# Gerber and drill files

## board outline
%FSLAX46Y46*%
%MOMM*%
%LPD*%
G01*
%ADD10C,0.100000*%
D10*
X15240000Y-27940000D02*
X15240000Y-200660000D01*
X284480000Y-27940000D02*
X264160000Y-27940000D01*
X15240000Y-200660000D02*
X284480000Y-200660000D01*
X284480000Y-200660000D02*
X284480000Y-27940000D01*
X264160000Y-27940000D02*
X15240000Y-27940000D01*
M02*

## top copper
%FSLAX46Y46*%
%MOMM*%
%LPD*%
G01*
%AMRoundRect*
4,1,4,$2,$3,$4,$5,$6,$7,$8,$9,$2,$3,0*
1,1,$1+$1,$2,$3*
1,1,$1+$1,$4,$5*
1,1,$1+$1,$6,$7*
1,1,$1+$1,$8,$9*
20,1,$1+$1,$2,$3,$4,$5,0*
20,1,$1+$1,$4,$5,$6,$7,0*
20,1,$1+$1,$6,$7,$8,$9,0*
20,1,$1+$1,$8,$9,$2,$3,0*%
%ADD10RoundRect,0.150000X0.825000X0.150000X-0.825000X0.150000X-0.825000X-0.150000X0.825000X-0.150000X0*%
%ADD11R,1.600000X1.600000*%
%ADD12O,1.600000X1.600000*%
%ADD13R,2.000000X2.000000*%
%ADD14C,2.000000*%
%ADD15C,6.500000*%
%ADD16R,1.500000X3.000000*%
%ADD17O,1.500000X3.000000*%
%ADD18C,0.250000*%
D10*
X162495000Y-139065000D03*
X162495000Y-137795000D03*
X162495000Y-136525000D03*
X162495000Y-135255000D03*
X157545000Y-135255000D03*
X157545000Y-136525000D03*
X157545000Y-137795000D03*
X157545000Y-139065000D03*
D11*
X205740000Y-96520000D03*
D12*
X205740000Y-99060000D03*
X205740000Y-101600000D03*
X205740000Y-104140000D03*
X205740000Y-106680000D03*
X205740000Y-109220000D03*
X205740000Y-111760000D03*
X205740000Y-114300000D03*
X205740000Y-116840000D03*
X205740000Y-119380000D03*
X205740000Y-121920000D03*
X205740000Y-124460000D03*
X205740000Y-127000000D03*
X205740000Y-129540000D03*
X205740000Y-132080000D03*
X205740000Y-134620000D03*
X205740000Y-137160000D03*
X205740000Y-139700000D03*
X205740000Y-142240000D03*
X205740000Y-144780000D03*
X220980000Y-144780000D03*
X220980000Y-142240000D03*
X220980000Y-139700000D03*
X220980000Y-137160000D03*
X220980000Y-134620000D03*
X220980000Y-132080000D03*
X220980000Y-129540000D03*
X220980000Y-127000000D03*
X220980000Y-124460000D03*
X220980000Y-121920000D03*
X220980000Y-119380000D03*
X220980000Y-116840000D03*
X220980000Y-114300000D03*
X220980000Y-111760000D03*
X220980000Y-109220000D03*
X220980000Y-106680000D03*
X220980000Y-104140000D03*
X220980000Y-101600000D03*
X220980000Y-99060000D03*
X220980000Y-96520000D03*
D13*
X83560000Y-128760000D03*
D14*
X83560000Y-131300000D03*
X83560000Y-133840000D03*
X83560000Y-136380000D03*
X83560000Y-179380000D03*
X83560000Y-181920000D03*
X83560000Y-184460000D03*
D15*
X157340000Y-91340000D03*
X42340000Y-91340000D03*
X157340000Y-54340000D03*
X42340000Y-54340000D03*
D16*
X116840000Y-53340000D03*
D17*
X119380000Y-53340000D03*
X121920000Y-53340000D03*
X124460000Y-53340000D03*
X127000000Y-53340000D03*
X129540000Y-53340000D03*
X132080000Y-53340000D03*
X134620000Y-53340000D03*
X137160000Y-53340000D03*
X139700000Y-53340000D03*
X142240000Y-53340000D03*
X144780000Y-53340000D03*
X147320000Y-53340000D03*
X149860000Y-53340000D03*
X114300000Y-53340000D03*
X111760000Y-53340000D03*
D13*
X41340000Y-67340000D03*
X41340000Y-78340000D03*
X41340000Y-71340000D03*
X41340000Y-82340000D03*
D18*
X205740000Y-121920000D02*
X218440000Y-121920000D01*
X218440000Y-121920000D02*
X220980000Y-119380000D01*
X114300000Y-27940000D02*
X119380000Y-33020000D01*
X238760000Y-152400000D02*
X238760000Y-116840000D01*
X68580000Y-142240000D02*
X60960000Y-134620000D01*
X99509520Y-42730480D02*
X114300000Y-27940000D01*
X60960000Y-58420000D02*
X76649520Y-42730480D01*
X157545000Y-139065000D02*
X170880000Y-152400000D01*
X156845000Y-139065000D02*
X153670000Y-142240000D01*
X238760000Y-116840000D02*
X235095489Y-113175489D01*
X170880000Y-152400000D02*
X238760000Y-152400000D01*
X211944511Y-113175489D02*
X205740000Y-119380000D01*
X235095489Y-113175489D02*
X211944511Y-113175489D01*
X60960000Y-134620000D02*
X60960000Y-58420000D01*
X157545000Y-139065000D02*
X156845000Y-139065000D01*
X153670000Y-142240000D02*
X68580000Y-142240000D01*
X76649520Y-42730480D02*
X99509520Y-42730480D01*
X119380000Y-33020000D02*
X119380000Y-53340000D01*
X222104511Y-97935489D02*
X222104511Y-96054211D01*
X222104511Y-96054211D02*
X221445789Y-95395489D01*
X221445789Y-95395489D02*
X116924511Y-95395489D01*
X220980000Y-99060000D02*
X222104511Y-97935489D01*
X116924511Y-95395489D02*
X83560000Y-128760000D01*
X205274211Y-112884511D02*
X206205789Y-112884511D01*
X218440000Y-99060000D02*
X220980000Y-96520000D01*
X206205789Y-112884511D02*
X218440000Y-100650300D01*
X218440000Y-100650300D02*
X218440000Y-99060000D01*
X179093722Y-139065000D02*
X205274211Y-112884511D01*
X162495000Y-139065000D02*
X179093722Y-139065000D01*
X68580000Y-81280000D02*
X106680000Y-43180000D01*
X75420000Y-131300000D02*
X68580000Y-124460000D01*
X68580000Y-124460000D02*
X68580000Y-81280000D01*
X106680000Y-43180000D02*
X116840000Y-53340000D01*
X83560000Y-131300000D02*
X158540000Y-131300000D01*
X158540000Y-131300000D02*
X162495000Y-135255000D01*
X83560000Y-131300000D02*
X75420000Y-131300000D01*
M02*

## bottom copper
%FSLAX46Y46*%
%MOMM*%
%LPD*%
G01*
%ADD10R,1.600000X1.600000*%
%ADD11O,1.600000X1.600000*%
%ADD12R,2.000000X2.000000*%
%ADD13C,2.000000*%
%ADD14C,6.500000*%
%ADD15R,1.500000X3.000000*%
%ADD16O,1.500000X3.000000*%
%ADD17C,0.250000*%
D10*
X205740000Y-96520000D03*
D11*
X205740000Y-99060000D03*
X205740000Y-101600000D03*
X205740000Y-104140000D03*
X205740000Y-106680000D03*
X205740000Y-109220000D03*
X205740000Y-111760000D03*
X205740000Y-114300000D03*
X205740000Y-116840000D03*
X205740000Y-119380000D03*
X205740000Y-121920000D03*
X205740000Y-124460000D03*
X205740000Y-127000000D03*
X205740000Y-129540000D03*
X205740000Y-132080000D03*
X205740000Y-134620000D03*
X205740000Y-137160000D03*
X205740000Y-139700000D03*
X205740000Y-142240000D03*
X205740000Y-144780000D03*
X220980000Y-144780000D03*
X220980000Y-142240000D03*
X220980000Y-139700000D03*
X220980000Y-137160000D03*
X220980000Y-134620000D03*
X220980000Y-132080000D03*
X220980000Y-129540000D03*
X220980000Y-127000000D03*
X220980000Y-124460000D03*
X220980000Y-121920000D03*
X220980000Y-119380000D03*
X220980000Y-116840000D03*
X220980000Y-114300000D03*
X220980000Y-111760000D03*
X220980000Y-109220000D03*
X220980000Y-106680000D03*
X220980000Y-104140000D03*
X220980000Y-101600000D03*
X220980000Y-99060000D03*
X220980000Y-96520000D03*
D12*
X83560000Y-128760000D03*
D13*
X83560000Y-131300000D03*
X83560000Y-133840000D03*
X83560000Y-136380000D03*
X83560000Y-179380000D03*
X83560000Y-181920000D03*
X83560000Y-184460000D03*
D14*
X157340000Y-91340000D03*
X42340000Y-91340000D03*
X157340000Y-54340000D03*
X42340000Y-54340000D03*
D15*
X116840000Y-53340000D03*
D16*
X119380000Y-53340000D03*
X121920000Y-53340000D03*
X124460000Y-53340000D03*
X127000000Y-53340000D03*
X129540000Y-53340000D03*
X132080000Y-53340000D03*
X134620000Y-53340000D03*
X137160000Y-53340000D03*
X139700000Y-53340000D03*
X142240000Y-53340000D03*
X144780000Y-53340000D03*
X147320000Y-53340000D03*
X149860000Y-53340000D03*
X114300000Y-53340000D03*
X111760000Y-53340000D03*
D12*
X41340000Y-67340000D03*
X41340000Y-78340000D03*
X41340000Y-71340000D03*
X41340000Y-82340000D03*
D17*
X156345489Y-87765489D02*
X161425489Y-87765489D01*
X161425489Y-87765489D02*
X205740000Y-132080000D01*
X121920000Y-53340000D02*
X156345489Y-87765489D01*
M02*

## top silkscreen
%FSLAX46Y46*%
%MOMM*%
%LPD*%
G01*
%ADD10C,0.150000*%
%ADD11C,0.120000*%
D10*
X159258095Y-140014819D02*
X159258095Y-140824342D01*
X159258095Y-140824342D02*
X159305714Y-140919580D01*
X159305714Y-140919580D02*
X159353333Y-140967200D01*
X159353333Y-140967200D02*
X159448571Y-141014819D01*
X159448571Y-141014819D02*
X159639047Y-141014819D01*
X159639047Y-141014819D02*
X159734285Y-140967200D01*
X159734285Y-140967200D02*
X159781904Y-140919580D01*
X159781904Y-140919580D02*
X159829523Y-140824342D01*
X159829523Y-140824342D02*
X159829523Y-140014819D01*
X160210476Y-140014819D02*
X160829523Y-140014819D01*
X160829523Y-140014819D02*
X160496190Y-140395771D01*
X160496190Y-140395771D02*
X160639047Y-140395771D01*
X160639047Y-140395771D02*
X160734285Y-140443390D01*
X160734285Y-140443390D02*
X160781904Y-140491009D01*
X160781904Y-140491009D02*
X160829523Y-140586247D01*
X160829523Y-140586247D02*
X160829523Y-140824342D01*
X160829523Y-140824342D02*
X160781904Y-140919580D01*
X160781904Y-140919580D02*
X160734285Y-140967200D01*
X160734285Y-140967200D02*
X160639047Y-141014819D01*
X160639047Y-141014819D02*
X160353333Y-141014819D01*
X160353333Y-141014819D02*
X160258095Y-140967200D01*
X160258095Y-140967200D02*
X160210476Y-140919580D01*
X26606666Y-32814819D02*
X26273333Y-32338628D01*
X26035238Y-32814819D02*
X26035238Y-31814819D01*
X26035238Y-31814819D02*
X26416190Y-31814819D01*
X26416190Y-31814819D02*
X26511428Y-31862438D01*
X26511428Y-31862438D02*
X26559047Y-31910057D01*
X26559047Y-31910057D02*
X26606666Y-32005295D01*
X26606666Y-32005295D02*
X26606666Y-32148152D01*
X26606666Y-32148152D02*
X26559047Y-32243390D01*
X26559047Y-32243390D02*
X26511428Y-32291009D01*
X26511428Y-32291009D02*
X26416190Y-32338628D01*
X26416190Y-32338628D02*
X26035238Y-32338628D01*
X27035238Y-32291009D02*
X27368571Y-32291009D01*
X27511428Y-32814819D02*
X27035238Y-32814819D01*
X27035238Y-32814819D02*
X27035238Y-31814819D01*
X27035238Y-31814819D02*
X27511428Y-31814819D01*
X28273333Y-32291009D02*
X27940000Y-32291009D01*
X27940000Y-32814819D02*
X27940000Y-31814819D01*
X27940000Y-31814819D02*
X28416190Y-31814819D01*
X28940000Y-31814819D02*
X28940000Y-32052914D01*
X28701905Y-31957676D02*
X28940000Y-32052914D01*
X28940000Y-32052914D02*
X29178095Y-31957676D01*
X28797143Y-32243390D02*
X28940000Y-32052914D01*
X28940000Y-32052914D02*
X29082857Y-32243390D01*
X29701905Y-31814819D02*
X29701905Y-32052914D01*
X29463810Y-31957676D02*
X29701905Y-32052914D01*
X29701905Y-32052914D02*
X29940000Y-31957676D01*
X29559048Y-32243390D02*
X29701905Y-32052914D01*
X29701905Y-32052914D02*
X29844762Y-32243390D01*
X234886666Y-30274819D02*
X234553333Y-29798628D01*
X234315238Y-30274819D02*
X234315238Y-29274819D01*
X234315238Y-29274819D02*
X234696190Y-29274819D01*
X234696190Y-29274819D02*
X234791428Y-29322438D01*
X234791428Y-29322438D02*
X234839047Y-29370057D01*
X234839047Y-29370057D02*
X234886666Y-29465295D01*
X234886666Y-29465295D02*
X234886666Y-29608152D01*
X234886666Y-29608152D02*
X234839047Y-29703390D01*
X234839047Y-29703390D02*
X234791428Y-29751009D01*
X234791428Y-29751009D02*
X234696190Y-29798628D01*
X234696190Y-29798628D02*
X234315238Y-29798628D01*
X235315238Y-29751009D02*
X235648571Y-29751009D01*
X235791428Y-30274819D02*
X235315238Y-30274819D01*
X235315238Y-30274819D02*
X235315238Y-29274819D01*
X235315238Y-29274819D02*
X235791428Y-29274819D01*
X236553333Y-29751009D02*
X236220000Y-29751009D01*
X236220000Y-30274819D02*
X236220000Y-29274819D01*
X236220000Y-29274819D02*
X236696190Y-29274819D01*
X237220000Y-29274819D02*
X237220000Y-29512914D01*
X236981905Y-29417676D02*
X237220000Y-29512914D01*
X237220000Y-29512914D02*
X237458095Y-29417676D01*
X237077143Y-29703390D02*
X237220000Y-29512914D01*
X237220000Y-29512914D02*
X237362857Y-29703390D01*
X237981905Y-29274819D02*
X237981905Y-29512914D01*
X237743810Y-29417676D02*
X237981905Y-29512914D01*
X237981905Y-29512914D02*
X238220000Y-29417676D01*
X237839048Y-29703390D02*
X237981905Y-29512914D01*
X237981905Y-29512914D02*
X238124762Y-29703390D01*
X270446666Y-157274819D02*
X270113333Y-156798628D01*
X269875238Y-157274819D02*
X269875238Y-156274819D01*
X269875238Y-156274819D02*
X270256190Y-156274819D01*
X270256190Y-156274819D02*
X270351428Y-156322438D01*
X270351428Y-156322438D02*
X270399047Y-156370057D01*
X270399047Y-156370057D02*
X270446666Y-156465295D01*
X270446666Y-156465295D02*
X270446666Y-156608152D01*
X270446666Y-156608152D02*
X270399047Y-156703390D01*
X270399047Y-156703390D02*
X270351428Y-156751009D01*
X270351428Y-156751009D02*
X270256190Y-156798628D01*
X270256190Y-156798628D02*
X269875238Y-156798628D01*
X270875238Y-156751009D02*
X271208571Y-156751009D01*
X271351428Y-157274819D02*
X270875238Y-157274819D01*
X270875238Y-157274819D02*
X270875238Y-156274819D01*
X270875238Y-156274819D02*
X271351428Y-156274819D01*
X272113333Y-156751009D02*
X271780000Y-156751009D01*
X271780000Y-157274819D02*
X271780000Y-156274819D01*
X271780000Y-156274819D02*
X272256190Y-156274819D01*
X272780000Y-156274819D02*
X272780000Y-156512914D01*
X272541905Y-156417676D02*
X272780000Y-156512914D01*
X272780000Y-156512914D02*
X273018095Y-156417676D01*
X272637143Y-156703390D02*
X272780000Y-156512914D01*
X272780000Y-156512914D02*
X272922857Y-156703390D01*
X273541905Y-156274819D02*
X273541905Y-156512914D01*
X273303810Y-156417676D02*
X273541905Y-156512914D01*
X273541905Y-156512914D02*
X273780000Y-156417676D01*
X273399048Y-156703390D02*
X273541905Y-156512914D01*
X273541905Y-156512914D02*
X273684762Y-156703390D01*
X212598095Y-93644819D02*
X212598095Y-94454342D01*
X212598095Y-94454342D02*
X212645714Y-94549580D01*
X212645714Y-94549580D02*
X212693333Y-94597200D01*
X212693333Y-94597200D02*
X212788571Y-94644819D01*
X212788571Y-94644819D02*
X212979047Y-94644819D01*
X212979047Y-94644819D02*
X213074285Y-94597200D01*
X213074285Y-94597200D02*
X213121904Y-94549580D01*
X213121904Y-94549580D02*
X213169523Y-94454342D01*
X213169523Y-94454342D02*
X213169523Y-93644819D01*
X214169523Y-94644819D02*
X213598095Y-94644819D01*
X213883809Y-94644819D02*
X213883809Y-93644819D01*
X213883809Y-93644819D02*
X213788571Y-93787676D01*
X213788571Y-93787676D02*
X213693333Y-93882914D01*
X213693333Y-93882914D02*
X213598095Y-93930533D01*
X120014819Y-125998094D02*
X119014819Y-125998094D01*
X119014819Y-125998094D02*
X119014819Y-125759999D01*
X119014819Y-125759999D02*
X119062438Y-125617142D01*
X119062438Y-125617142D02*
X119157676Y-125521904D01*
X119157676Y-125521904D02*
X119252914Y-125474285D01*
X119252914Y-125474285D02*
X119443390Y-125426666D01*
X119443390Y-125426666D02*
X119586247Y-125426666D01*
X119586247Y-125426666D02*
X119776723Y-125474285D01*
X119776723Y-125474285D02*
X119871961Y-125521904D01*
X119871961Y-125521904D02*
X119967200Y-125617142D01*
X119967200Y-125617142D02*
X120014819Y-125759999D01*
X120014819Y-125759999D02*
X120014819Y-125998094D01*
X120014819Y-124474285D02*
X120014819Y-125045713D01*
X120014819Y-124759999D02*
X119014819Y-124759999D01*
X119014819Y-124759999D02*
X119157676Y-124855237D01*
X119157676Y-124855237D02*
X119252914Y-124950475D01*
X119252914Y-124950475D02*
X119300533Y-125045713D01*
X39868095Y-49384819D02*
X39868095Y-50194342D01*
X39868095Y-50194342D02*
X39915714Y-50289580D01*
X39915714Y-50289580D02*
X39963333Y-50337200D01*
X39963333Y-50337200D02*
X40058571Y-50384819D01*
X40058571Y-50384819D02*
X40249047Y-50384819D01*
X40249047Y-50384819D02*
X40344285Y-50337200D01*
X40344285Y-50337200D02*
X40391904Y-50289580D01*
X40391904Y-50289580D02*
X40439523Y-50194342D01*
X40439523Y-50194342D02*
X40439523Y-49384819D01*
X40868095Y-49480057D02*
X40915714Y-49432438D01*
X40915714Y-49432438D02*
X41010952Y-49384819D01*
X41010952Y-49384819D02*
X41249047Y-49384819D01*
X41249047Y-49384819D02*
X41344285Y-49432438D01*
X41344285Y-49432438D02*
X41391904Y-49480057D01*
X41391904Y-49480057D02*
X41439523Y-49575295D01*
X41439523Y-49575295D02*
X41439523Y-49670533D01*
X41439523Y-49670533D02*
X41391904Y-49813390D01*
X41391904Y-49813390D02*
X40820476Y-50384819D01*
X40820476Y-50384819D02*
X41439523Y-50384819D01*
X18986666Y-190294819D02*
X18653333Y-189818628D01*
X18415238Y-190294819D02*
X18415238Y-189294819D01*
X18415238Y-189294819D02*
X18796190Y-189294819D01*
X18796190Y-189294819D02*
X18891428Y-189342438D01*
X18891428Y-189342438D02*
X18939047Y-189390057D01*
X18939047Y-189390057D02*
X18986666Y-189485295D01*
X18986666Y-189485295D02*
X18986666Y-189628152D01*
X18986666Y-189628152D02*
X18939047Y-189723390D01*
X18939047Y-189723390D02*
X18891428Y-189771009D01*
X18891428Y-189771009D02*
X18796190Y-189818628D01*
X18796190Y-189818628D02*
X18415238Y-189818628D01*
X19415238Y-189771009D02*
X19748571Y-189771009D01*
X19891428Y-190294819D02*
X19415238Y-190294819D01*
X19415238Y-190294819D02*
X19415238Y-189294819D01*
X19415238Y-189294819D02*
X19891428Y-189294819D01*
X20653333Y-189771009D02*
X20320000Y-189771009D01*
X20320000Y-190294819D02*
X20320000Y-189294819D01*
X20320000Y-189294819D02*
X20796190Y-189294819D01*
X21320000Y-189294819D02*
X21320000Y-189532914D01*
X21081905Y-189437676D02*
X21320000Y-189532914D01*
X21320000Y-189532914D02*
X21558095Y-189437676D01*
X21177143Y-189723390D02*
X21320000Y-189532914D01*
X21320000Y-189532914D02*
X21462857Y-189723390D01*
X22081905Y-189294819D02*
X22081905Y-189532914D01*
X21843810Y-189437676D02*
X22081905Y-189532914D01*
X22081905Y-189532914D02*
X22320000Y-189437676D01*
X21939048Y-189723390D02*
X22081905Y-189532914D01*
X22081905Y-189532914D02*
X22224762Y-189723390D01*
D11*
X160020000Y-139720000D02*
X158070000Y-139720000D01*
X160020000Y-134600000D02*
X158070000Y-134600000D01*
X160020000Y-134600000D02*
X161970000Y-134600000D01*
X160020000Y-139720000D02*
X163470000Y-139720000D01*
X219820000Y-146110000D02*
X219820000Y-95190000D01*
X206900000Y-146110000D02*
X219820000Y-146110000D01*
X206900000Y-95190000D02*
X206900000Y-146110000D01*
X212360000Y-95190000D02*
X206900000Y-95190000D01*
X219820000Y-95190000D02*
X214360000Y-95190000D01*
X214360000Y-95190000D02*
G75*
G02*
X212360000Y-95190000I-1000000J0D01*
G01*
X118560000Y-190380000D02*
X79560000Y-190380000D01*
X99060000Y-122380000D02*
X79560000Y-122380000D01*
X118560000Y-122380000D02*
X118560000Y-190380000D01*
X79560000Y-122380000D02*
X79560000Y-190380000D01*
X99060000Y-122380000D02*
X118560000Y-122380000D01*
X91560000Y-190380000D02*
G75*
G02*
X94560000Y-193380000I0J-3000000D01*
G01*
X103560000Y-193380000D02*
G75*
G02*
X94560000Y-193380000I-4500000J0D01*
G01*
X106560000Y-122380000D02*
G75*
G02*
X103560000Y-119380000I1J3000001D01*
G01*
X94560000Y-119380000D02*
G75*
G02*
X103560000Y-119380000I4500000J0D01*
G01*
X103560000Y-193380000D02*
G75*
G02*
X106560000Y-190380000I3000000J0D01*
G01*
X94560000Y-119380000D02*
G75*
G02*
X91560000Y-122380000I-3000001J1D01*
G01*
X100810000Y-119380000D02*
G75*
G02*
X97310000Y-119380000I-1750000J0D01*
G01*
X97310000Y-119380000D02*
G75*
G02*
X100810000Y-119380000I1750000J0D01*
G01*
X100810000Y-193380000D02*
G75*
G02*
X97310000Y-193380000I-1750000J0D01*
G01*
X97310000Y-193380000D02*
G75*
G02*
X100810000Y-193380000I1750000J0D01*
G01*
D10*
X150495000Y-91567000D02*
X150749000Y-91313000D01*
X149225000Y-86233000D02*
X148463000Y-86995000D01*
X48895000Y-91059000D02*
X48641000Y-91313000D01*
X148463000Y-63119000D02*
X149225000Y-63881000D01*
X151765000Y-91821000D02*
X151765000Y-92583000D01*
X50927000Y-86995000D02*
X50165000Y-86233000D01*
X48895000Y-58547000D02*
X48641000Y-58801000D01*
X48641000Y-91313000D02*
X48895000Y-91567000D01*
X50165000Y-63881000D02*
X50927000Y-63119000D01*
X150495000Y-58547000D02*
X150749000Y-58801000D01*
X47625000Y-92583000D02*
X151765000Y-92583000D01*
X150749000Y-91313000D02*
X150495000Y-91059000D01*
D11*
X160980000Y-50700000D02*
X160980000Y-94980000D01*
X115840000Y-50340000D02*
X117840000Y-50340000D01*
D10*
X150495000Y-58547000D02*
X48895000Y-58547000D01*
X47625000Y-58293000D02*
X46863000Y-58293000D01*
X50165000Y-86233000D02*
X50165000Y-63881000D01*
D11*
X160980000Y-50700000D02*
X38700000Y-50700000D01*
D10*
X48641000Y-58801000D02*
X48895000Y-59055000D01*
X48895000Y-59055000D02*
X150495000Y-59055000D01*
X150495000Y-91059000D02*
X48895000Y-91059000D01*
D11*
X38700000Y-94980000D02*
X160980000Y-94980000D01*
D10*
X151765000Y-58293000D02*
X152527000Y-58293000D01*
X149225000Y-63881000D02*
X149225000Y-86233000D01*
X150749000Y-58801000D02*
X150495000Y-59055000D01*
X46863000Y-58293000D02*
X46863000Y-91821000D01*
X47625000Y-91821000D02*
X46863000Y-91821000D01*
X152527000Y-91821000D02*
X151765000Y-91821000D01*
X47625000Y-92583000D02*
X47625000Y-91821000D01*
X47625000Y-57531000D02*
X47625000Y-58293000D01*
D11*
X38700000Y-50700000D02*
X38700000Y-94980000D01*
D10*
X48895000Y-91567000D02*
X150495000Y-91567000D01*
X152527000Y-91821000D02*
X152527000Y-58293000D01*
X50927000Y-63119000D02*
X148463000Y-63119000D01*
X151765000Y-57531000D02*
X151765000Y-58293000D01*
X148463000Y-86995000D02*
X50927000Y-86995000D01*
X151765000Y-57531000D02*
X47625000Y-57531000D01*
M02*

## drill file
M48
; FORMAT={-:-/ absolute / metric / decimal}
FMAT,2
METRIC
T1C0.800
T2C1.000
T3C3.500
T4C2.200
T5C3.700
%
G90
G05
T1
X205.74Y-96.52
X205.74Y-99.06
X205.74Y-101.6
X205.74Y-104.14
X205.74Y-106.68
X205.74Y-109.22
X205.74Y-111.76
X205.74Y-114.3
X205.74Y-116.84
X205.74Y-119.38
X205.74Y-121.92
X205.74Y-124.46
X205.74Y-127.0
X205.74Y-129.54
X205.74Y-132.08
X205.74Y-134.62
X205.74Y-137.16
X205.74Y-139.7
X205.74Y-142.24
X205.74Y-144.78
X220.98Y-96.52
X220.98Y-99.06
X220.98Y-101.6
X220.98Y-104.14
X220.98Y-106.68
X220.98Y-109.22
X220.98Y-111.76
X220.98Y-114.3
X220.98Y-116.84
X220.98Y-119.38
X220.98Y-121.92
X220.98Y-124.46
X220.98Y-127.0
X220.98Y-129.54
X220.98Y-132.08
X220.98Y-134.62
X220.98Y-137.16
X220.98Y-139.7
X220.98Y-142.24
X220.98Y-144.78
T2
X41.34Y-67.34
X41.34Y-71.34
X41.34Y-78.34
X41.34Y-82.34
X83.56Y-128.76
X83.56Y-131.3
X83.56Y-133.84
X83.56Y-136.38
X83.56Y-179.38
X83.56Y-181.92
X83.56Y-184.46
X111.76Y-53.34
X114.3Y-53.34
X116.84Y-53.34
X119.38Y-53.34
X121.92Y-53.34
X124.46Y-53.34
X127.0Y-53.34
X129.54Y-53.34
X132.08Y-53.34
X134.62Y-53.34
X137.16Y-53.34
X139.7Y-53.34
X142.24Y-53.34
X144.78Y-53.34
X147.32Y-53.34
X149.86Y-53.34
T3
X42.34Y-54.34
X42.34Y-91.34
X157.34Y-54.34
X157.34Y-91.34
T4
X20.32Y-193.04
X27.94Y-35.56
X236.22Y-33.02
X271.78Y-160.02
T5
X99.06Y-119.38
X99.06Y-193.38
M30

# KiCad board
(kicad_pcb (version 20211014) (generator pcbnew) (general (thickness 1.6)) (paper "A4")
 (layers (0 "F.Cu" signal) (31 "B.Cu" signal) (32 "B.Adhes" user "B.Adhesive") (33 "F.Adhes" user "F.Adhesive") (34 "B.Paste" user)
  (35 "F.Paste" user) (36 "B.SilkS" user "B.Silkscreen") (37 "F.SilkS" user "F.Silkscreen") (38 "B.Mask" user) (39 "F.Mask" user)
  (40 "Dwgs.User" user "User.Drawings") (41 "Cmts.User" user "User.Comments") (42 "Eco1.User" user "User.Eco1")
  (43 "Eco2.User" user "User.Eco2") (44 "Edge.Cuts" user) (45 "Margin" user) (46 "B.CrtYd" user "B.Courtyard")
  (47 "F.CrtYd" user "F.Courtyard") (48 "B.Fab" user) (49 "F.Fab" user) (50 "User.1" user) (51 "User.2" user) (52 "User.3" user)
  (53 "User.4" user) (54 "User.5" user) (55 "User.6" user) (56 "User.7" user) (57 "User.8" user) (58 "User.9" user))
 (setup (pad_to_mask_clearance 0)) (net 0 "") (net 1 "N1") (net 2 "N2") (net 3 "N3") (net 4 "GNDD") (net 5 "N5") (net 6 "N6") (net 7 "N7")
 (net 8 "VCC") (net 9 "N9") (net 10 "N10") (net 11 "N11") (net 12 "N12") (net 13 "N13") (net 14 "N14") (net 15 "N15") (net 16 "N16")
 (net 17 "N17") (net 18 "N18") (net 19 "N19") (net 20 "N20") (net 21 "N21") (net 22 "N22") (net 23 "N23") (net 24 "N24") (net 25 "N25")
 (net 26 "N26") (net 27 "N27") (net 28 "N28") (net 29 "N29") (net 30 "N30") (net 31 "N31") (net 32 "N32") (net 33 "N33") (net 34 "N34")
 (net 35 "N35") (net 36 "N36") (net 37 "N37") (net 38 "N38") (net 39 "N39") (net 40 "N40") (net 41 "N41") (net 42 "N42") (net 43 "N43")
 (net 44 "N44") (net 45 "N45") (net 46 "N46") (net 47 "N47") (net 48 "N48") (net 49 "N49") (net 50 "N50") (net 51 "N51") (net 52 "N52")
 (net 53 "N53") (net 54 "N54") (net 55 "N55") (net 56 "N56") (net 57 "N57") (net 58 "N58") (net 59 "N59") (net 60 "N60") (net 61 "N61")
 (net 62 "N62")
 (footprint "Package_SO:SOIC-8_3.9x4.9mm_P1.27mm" (layer "F.Cu") (at 160.02 137.16 180)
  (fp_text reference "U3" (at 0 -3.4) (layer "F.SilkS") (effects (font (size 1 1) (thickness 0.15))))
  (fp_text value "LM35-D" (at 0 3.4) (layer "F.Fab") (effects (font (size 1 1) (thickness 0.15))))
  (fp_line (start 0 -2.56) (end 1.95 -2.56) (layer "F.SilkS") (width 0.12))
  (fp_line (start 0 2.56) (end 1.95 2.56) (layer "F.SilkS") (width 0.12))
  (fp_line (start 0 2.56) (end -1.95 2.56) (layer "F.SilkS") (width 0.12))
  (fp_line (start 0 -2.56) (end -3.45 -2.56) (layer "F.SilkS") (width 0.12))
  (pad "1" smd roundrect (at -2.475 -1.905 180) (size 1.95 0.6) (layers "F.Cu" "F.Paste" "F.Mask") (roundrect_rratio 0.25) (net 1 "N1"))
  (pad "2" smd roundrect (at -2.475 -0.635 180) (size 1.95 0.6) (layers "F.Cu" "F.Paste" "F.Mask") (roundrect_rratio 0.25) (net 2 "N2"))
  (pad "3" smd roundrect (at -2.475 0.635 180) (size 1.95 0.6) (layers "F.Cu" "F.Paste" "F.Mask") (roundrect_rratio 0.25) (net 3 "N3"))
  (pad "4" smd roundrect (at -2.475 1.905 180) (size 1.95 0.6) (layers "F.Cu" "F.Paste" "F.Mask") (roundrect_rratio 0.25) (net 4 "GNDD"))
  (pad "5" smd roundrect (at 2.475 1.905 180) (size 1.95 0.6) (layers "F.Cu" "F.Paste" "F.Mask") (roundrect_rratio 0.25) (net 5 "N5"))
  (pad "6" smd roundrect (at 2.475 0.635 180) (size 1.95 0.6) (layers "F.Cu" "F.Paste" "F.Mask") (roundrect_rratio 0.25) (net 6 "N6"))
  (pad "7" smd roundrect (at 2.475 -0.635 180) (size 1.95 0.6) (layers "F.Cu" "F.Paste" "F.Mask") (roundrect_rratio 0.25) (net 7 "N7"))
  (pad "8" smd roundrect (at 2.475 -1.905 180) (size 1.95 0.6) (layers "F.Cu" "F.Paste" "F.Mask") (roundrect_rratio 0.25) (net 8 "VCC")))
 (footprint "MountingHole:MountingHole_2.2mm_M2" (layer "F.Cu") (at 27.94 35.56)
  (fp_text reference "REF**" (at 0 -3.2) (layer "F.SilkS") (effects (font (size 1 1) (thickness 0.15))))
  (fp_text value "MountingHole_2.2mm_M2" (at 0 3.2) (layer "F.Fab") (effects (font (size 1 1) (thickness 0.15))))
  (pad "" np_thru_hole circle (at 0 0) (size 2.2 2.2) (drill 2.2) (layers *.Cu *.Mask)))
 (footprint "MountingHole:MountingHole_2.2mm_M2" (layer "F.Cu") (at 236.22 33.02)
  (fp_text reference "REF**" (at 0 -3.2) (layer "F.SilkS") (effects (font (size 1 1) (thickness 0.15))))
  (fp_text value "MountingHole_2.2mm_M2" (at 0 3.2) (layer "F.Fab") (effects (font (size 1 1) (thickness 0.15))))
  (pad "" np_thru_hole circle (at 0 0) (size 2.2 2.2) (drill 2.2) (layers *.Cu *.Mask)))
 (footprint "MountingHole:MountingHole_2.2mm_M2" (layer "F.Cu") (at 271.78 160.02)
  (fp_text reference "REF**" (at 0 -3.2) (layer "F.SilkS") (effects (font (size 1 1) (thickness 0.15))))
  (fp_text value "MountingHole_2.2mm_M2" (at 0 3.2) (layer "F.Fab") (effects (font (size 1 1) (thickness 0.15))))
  (pad "" np_thru_hole circle (at 0 0) (size 2.2 2.2) (drill 2.2) (layers *.Cu *.Mask)))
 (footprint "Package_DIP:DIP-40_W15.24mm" (layer "F.Cu") (at 205.74 96.52)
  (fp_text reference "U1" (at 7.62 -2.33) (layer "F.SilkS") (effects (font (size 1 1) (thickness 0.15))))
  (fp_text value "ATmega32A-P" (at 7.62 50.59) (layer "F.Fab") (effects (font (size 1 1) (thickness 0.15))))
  (fp_line (start 14.08 49.59) (end 14.08 -1.33) (layer "F.SilkS") (width 0.12))
  (fp_line (start 1.16 49.59) (end 14.08 49.59) (layer "F.SilkS") (width 0.12))
  (fp_line (start 1.16 -1.33) (end 1.16 49.59) (layer "F.SilkS") (width 0.12))
  (fp_line (start 6.62 -1.33) (end 1.16 -1.33) (layer "F.SilkS") (width 0.12))
  (fp_line (start 14.08 -1.33) (end 8.62 -1.33) (layer "F.SilkS") (width 0.12))
  (fp_arc (start 8.62 -1.33) (mid 7.62 -0.33) (end 6.62 -1.33) (layer "F.SilkS") (width 0.12))
  (pad "1" thru_hole rect (at 0 0) (size 1.6 1.6) (drill 0.8) (layers *.Cu *.Mask) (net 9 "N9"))
  (pad "2" thru_hole oval (at 0 2.54) (size 1.6 1.6) (drill 0.8) (layers *.Cu *.Mask) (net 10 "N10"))
  (pad "3" thru_hole oval (at 0 5.08) (size 1.6 1.6) (drill 0.8) (layers *.Cu *.Mask) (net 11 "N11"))
  (pad "4" thru_hole oval (at 0 7.62) (size 1.6 1.6) (drill 0.8) (layers *.Cu *.Mask) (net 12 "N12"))
  (pad "5" thru_hole oval (at 0 10.16) (size 1.6 1.6) (drill 0.8) (layers *.Cu *.Mask) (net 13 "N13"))
  (pad "6" thru_hole oval (at 0 12.7) (size 1.6 1.6) (drill 0.8) (layers *.Cu *.Mask) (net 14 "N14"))
  (pad "7" thru_hole oval (at 0 15.24) (size 1.6 1.6) (drill 0.8) (layers *.Cu *.Mask) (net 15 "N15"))
  (pad "8" thru_hole oval (at 0 17.78) (size 1.6 1.6) (drill 0.8) (layers *.Cu *.Mask) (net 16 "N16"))
  (pad "9" thru_hole oval (at 0 20.32) (size 1.6 1.6) (drill 0.8) (layers *.Cu *.Mask) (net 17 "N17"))
  (pad "10" thru_hole oval (at 0 22.86) (size 1.6 1.6) (drill 0.8) (layers *.Cu *.Mask) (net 8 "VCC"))
  (pad "11" thru_hole oval (at 0 25.4) (size 1.6 1.6) (drill 0.8) (layers *.Cu *.Mask) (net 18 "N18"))
  (pad "12" thru_hole oval (at 0 27.94) (size 1.6 1.6) (drill 0.8) (layers *.Cu *.Mask) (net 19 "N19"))
  (pad "13" thru_hole oval (at 0 30.48) (size 1.6 1.6) (drill 0.8) (layers *.Cu *.Mask) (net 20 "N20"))
  (pad "14" thru_hole oval (at 0 33.02) (size 1.6 1.6) (drill 0.8) (layers *.Cu *.Mask) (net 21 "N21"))
  (pad "15" thru_hole oval (at 0 35.56) (size 1.6 1.6) (drill 0.8) (layers *.Cu *.Mask) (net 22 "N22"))
  (pad "16" thru_hole oval (at 0 38.1) (size 1.6 1.6) (drill 0.8) (layers *.Cu *.Mask) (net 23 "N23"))
  (pad "17" thru_hole oval (at 0 40.64) (size 1.6 1.6) (drill 0.8) (layers *.Cu *.Mask) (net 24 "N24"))
  (pad "18" thru_hole oval (at 0 43.18) (size 1.6 1.6) (drill 0.8) (layers *.Cu *.Mask) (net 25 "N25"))
  (pad "19" thru_hole oval (at 0 45.72) (size 1.6 1.6) (drill 0.8) (layers *.Cu *.Mask) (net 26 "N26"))
  (pad "20" thru_hole oval (at 0 48.26) (size 1.6 1.6) (drill 0.8) (layers *.Cu *.Mask) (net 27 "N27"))
  (pad "21" thru_hole oval (at 15.24 48.26) (size 1.6 1.6) (drill 0.8) (layers *.Cu *.Mask) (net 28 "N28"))
  (pad "22" thru_hole oval (at 15.24 45.72) (size 1.6 1.6) (drill 0.8) (layers *.Cu *.Mask) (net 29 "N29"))
  (pad "23" thru_hole oval (at 15.24 43.18) (size 1.6 1.6) (drill 0.8) (layers *.Cu *.Mask) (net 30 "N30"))
  (pad "24" thru_hole oval (at 15.24 40.64) (size 1.6 1.6) (drill 0.8) (layers *.Cu *.Mask) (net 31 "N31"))
  (pad "25" thru_hole oval (at 15.24 38.1) (size 1.6 1.6) (drill 0.8) (layers *.Cu *.Mask) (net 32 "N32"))
  (pad "26" thru_hole oval (at 15.24 35.56) (size 1.6 1.6) (drill 0.8) (layers *.Cu *.Mask) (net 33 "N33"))
  (pad "27" thru_hole oval (at 15.24 33.02) (size 1.6 1.6) (drill 0.8) (layers *.Cu *.Mask) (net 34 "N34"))
  (pad "28" thru_hole oval (at 15.24 30.48) (size 1.6 1.6) (drill 0.8) (layers *.Cu *.Mask) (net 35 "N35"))
  (pad "29" thru_hole oval (at 15.24 27.94) (size 1.6 1.6) (drill 0.8) (layers *.Cu *.Mask) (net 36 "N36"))
  (pad "30" thru_hole oval (at 15.24 25.4) (size 1.6 1.6) (drill 0.8) (layers *.Cu *.Mask) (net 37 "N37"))
  (pad "31" thru_hole oval (at 15.24 22.86) (size 1.6 1.6) (drill 0.8) (layers *.Cu *.Mask) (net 18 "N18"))
  (pad "32" thru_hole oval (at 15.24 20.32) (size 1.6 1.6) (drill 0.8) (layers *.Cu *.Mask) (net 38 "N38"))
  (pad "33" thru_hole oval (at 15.24 17.78) (size 1.6 1.6) (drill 0.8) (layers *.Cu *.Mask) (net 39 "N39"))
  (pad "34" thru_hole oval (at 15.24 15.24) (size 1.6 1.6) (drill 0.8) (layers *.Cu *.Mask) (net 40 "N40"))
  (pad "35" thru_hole oval (at 15.24 12.7) (size 1.6 1.6) (drill 0.8) (layers *.Cu *.Mask) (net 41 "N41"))
  (pad "36" thru_hole oval (at 15.24 10.16) (size 1.6 1.6) (drill 0.8) (layers *.Cu *.Mask) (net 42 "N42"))
  (pad "37" thru_hole oval (at 15.24 7.62) (size 1.6 1.6) (drill 0.8) (layers *.Cu *.Mask) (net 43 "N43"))
  (pad "38" thru_hole oval (at 15.24 5.08) (size 1.6 1.6) (drill 0.8) (layers *.Cu *.Mask) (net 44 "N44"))
  (pad "39" thru_hole oval (at 15.24 2.54) (size 1.6 1.6) (drill 0.8) (layers *.Cu *.Mask) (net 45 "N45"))
  (pad "40" thru_hole oval (at 15.24 0) (size 1.6 1.6) (drill 0.8) (layers *.Cu *.Mask) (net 1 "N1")))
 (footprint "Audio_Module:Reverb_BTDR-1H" (layer "F.Cu") (at 83.56 128.76 -90)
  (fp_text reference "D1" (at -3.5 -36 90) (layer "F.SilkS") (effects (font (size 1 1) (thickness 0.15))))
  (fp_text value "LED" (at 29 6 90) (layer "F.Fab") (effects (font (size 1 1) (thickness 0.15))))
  (fp_line (start 61.62 -35) (end 61.62 4) (layer "F.SilkS") (width 0.12))
  (fp_line (start -6.38 -15.5) (end -6.38 4) (layer "F.SilkS") (width 0.12))
  (fp_line (start -6.38 -35) (end 61.62 -35) (layer "F.SilkS") (width 0.12))
  (fp_line (start -6.38 4) (end 61.62 4) (layer "F.SilkS") (width 0.12))
  (fp_line (start -6.38 -15.5) (end -6.38 -35) (layer "F.SilkS") (width 0.12))
  (fp_arc (start 61.62 -8) (mid 62.49868 -10.12132) (end 64.62 -11) (layer "F.SilkS") (width 0.12))
  (fp_arc (start 64.62 -20) (mid 69.12 -15.5) (end 64.62 -11) (layer "F.SilkS") (width 0.12))
  (fp_arc (start -6.38 -23) (mid -7.25868 -20.87868) (end -9.38 -20) (layer "F.SilkS") (width 0.12))
  (fp_arc (start -9.38 -11) (mid -13.88 -15.5) (end -9.38 -20) (layer "F.SilkS") (width 0.12))
  (fp_arc (start 64.62 -20) (mid 62.49868 -20.87868) (end 61.62 -23) (layer "F.SilkS") (width 0.12))
  (fp_arc (start -9.38 -11) (mid -7.25868 -10.12132) (end -6.38 -8) (layer "F.SilkS") (width 0.12))
  (fp_circle (center -9.38 -15.5) (end -7.63 -15.5) (layer "F.SilkS") (width 0.12) (fill none))
  (fp_circle (center 64.62 -15.5) (end 66.37 -15.5) (layer "F.SilkS") (width 0.12) (fill none))
  (pad "" np_thru_hole circle (at 64.62 -15.5 270) (size 3.7 3.7) (drill 3.7) (layers *.Cu *.Mask))
  (pad "" np_thru_hole circle (at -9.38 -15.5 270) (size 3.7 3.7) (drill 3.7) (layers *.Cu *.Mask))
  (pad "1" thru_hole rect (at 0 0 270) (size 2 2) (drill 1) (layers *.Cu *.Mask) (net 45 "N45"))
  (pad "2" thru_hole circle (at 2.54 0 270) (size 2 2) (drill 1) (layers *.Cu *.Mask) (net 4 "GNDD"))
  (pad "3" thru_hole circle (at 5.08 0 270) (size 2 2) (drill 1) (layers *.Cu *.Mask))
  (pad "4" thru_hole circle (at 7.62 0 270) (size 2 2) (drill 1) (layers *.Cu *.Mask))
  (pad "5" thru_hole circle (at 50.62 0 270) (size 2 2) (drill 1) (layers *.Cu *.Mask))
  (pad "6" thru_hole circle (at 53.16 0 270) (size 2 2) (drill 1) (layers *.Cu *.Mask))
  (pad "7" thru_hole circle (at 55.7 0 270) (size 2 2) (drill 1) (layers *.Cu *.Mask)))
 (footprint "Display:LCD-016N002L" (layer "F.Cu") (at 116.84 53.34)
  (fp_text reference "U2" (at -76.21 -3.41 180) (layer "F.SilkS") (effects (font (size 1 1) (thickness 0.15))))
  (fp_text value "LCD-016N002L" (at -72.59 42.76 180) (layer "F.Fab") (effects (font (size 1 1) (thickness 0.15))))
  (fp_line (start 33.655 38.227) (end 33.909 37.973) (layer "F.SilkS") (width 0.15))
  (fp_line (start 32.385 32.893) (end 31.623 33.655) (layer "F.SilkS") (width 0.15))
  (fp_line (start -67.945 37.719) (end -68.199 37.973) (layer "F.SilkS") (width 0.15))
  (fp_line (start 31.623 9.779) (end 32.385 10.541) (layer "F.SilkS") (width 0.15))
  (fp_line (start 34.925 38.481) (end 34.925 39.243) (layer "F.SilkS") (width 0.15))
  (fp_line (start -65.913 33.655) (end -66.675 32.893) (layer "F.SilkS") (width 0.15))
  (fp_line (start -67.945 5.207) (end -68.199 5.461) (layer "F.SilkS") (width 0.15))
  (fp_line (start -68.199 37.973) (end -67.945 38.227) (layer "F.SilkS") (width 0.15))
  (fp_line (start -66.675 10.541) (end -65.913 9.779) (layer "F.SilkS") (width 0.15))
  (fp_line (start 33.655 5.207) (end 33.909 5.461) (layer "F.SilkS") (width 0.15))
  (fp_line (start -69.215 39.243) (end 34.925 39.243) (layer "F.SilkS") (width 0.15))
  (fp_line (start 33.909 37.973) (end 33.655 37.719) (layer "F.SilkS") (width 0.15))
  (fp_line (start 44.14 -2.64) (end 44.14 41.64) (layer "F.SilkS") (width 0.12))
  (fp_line (start -1 -3) (end 1 -3) (layer "F.SilkS") (width 0.12))
  (fp_line (start 33.655 5.207) (end -67.945 5.207) (layer "F.SilkS") (width 0.15))
  (fp_line (start -69.215 4.953) (end -69.977 4.953) (layer "F.SilkS") (width 0.15))
  (fp_line (start -66.675 32.893) (end -66.675 10.541) (layer "F.SilkS") (width 0.15))
  (fp_line (start 44.14 -2.64) (end -78.14 -2.64) (layer "F.SilkS") (width 0.12))
  (fp_line (start -68.199 5.461) (end -67.945 5.715) (layer "F.SilkS") (width 0.15))
  (fp_line (start -67.945 5.715) (end 33.655 5.715) (layer "F.SilkS") (width 0.15))
  (fp_line (start 33.655 37.719) (end -67.945 37.719) (layer "F.SilkS") (width 0.15))
  (fp_line (start -78.14 41.64) (end 44.14 41.64) (layer "F.SilkS") (width 0.12))
  (fp_line (start 34.925 4.953) (end 35.687 4.953) (layer "F.SilkS") (width 0.15))
  (fp_line (start 32.385 10.541) (end 32.385 32.893) (layer "F.SilkS") (width 0.15))
  (fp_line (start 33.909 5.461) (end 33.655 5.715) (layer "F.SilkS") (width 0.15))
  (fp_line (start -69.977 4.953) (end -69.977 38.481) (layer "F.SilkS") (width 0.15))
  (fp_line (start -69.215 38.481) (end -69.977 38.481) (layer "F.SilkS") (width 0.15))
  (fp_line (start 35.687 38.481) (end 34.925 38.481) (layer "F.SilkS") (width 0.15))
  (fp_line (start -69.215 39.243) (end -69.215 38.481) (layer "F.SilkS") (width 0.15))
  (fp_line (start -69.215 4.191) (end -69.215 4.953) (layer "F.SilkS") (width 0.15))
  (fp_line (start -78.14 -2.64) (end -78.14 41.64) (layer "F.SilkS") (width 0.12))
  (fp_line (start -67.945 38.227) (end 33.655 38.227) (layer "F.SilkS") (width 0.15))
  (fp_line (start 35.687 38.481) (end 35.687 4.953) (layer "F.SilkS") (width 0.15))
  (fp_line (start -65.913 9.779) (end 31.623 9.779) (layer "F.SilkS") (width 0.15))
  (fp_line (start 34.925 4.191) (end 34.925 4.953) (layer "F.SilkS") (width 0.15))
  (fp_line (start 31.623 33.655) (end -65.913 33.655) (layer "F.SilkS") (width 0.15))
  (fp_line (start 34.925 4.191) (end -69.215 4.191) (layer "F.SilkS") (width 0.15))
  (pad "" thru_hole circle (at 40.5 38 180) (size 6.5 6.5) (drill 3.5) (layers *.Cu *.Mask))
  (pad "" thru_hole circle (at -74.5 38 180) (size 6.5 6.5) (drill 3.5) (layers *.Cu *.Mask))
  (pad "" thru_hole circle (at 40.5 1 180) (size 6.5 6.5) (drill 3.5) (layers *.Cu *.Mask))
  (pad "" thru_hole circle (at -74.5 1 180) (size 6.5 6.5) (drill 3.5) (layers *.Cu *.Mask))
  (pad "1" thru_hole rect (at 0 0 180) (size 1.5 3) (drill 1) (layers *.Cu *.Mask) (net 4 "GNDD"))
  (pad "2" thru_hole oval (at 2.54 0 180) (size 1.5 3) (drill 1) (layers *.Cu *.Mask) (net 8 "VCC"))
  (pad "3" thru_hole oval (at 5.08 0 180) (size 1.5 3) (drill 1) (layers *.Cu *.Mask) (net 22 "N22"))
  (pad "4" thru_hole oval (at 7.62 0 180) (size 1.5 3) (drill 1) (layers *.Cu *.Mask) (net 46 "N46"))
  (pad "5" thru_hole oval (at 10.16 0 180) (size 1.5 3) (drill 1) (layers *.Cu *.Mask) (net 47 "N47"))
  (pad "6" thru_hole oval (at 12.7 0 180) (size 1.5 3) (drill 1) (layers *.Cu *.Mask) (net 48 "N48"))
  (pad "7" thru_hole oval (at 15.24 0 180) (size 1.5 3) (drill 1) (layers *.Cu *.Mask) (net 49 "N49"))
  (pad "8" thru_hole oval (at 17.78 0 180) (size 1.5 3) (drill 1) (layers *.Cu *.Mask) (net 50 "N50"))
  (pad "9" thru_hole oval (at 20.32 0 180) (size 1.5 3) (drill 1) (layers *.Cu *.Mask) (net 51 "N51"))
  (pad "10" thru_hole oval (at 22.86 0 180) (size 1.5 3) (drill 1) (layers *.Cu *.Mask) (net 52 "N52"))
  (pad "11" thru_hole oval (at 25.4 0 180) (size 1.5 3) (drill 1) (layers *.Cu *.Mask) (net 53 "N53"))
  (pad "12" thru_hole oval (at 27.94 0 180) (size 1.5 3) (drill 1) (layers *.Cu *.Mask) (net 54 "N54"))
  (pad "13" thru_hole oval (at 30.48 0 180) (size 1.5 3) (drill 1) (layers *.Cu *.Mask) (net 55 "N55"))
  (pad "14" thru_hole oval (at 33.02 0 180) (size 1.5 3) (drill 1) (layers *.Cu *.Mask) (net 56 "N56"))
  (pad "15" thru_hole oval (at -2.54 0 180) (size 1.5 3) (drill 1) (layers *.Cu *.Mask) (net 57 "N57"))
  (pad "16" thru_hole oval (at -5.08 0 180) (size 1.5 3) (drill 1) (layers *.Cu *.Mask) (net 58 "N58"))
  (pad "A1" thru_hole rect (at -75.5 14 180) (size 2 2) (drill 1) (layers *.Cu *.Mask) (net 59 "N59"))
  (pad "A2" thru_hole rect (at -75.5 25 180) (size 2 2) (drill 1) (layers *.Cu *.Mask) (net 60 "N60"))
  (pad "K1" thru_hole rect (at -75.5 18 180) (size 2 2) (drill 1) (layers *.Cu *.Mask) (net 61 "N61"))
  (pad "K2" thru_hole rect (at -75.5 29 180) (size 2 2) (drill 1) (layers *.Cu *.Mask) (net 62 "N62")))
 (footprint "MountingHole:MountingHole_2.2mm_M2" (layer "F.Cu") (at 20.32 193.04)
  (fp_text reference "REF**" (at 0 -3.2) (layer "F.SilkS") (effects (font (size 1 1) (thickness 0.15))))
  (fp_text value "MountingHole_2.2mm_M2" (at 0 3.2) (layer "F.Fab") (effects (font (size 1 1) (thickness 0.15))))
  (pad "" np_thru_hole circle (at 0 0) (size 2.2 2.2) (drill 2.2) (layers *.Cu *.Mask)))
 (gr_line (start 15.24 27.94) (end 15.24 200.66) (layer "Edge.Cuts") (width 0.1))
 (gr_line (start 284.48 27.94) (end 264.16 27.94) (layer "Edge.Cuts") (width 0.1))
 (gr_line (start 15.24 200.66) (end 284.48 200.66) (layer "Edge.Cuts") (width 0.1))
 (gr_line (start 284.48 200.66) (end 284.48 27.94) (layer "Edge.Cuts") (width 0.1))
 (gr_line (start 264.16 27.94) (end 15.24 27.94) (layer "Edge.Cuts") (width 0.1))
 (segment (start 205.74 121.92) (end 218.44 121.92) (width 0.25) (layer "F.Cu") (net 18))
 (segment (start 218.44 121.92) (end 220.98 119.38) (width 0.25) (layer "F.Cu") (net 18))
 (segment (start 156.345489 87.765489) (end 161.425489 87.765489) (width 0.25) (layer "B.Cu") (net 22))
 (segment (start 161.425489 87.765489) (end 205.74 132.08) (width 0.25) (layer "B.Cu") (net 22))
 (segment (start 121.92 53.34) (end 156.345489 87.765489) (width 0.25) (layer "B.Cu") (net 22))
 (segment (start 114.3 27.94) (end 119.38 33.02) (width 0.25) (layer "F.Cu") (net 8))
 (segment (start 238.76 152.4) (end 238.76 116.84) (width 0.25) (layer "F.Cu") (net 8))
 (segment (start 68.58 142.24) (end 60.96 134.62) (width 0.25) (layer "F.Cu") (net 8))
 (segment (start 99.50952 42.73048) (end 114.3 27.94) (width 0.25) (layer "F.Cu") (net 8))
 (segment (start 60.96 58.42) (end 76.64952 42.73048) (width 0.25) (layer "F.Cu") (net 8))
 (segment (start 157.545 139.065) (end 170.88 152.4) (width 0.25) (layer "F.Cu") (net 8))
 (segment (start 156.845 139.065) (end 153.67 142.24) (width 0.25) (layer "F.Cu") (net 8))
 (segment (start 238.76 116.84) (end 235.095489 113.175489) (width 0.25) (layer "F.Cu") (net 8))
 (segment (start 170.88 152.4) (end 238.76 152.4) (width 0.25) (layer "F.Cu") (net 8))
 (segment (start 211.944511 113.175489) (end 205.74 119.38) (width 0.25) (layer "F.Cu") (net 8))
 (segment (start 235.095489 113.175489) (end 211.944511 113.175489) (width 0.25) (layer "F.Cu") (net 8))
 (segment (start 60.96 134.62) (end 60.96 58.42) (width 0.25) (layer "F.Cu") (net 8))
 (segment (start 157.545 139.065) (end 156.845 139.065) (width 0.25) (layer "F.Cu") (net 8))
 (segment (start 153.67 142.24) (end 68.58 142.24) (width 0.25) (layer "F.Cu") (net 8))
 (segment (start 76.64952 42.73048) (end 99.50952 42.73048) (width 0.25) (layer "F.Cu") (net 8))
 (segment (start 119.38 33.02) (end 119.38 53.34) (width 0.25) (layer "F.Cu") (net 8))
 (segment (start 222.104511 97.935489) (end 222.104511 96.054211) (width 0.25) (layer "F.Cu") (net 45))
 (segment (start 222.104511 96.054211) (end 221.445789 95.395489) (width 0.25) (layer "F.Cu") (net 45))
 (segment (start 221.445789 95.395489) (end 116.924511 95.395489) (width 0.25) (layer "F.Cu") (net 45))
 (segment (start 220.98 99.06) (end 222.104511 97.935489) (width 0.25) (layer "F.Cu") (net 45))
 (segment (start 116.924511 95.395489) (end 83.56 128.76) (width 0.25) (layer "F.Cu") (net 45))
 (segment (start 205.274211 112.884511) (end 206.205789 112.884511) (width 0.25) (layer "F.Cu") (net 1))
 (segment (start 218.44 99.06) (end 220.98 96.52) (width 0.25) (layer "F.Cu") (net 1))
 (segment (start 206.205789 112.884511) (end 218.44 100.6503) (width 0.25) (layer "F.Cu") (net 1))
 (segment (start 218.44 100.6503) (end 218.44 99.06) (width 0.25) (layer "F.Cu") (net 1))
 (segment (start 179.093722 139.065) (end 205.274211 112.884511) (width 0.25) (layer "F.Cu") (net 1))
 (segment (start 162.495 139.065) (end 179.093722 139.065) (width 0.25) (layer "F.Cu") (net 1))
 (segment (start 68.58 81.28) (end 106.68 43.18) (width 0.25) (layer "F.Cu") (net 4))
 (segment (start 75.42 131.3) (end 68.58 124.46) (width 0.25) (layer "F.Cu") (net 4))
 (segment (start 68.58 124.46) (end 68.58 81.28) (width 0.25) (layer "F.Cu") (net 4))
 (segment (start 106.68 43.18) (end 116.84 53.34) (width 0.25) (layer "F.Cu") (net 4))
 (segment (start 83.56 131.3) (end 158.54 131.3) (width 0.25) (layer "F.Cu") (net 4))
 (segment (start 158.54 131.3) (end 162.495 135.255) (width 0.25) (layer "F.Cu") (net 4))
 (segment (start 83.56 131.3) (end 75.42 131.3) (width 0.25) (layer "F.Cu") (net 4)))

